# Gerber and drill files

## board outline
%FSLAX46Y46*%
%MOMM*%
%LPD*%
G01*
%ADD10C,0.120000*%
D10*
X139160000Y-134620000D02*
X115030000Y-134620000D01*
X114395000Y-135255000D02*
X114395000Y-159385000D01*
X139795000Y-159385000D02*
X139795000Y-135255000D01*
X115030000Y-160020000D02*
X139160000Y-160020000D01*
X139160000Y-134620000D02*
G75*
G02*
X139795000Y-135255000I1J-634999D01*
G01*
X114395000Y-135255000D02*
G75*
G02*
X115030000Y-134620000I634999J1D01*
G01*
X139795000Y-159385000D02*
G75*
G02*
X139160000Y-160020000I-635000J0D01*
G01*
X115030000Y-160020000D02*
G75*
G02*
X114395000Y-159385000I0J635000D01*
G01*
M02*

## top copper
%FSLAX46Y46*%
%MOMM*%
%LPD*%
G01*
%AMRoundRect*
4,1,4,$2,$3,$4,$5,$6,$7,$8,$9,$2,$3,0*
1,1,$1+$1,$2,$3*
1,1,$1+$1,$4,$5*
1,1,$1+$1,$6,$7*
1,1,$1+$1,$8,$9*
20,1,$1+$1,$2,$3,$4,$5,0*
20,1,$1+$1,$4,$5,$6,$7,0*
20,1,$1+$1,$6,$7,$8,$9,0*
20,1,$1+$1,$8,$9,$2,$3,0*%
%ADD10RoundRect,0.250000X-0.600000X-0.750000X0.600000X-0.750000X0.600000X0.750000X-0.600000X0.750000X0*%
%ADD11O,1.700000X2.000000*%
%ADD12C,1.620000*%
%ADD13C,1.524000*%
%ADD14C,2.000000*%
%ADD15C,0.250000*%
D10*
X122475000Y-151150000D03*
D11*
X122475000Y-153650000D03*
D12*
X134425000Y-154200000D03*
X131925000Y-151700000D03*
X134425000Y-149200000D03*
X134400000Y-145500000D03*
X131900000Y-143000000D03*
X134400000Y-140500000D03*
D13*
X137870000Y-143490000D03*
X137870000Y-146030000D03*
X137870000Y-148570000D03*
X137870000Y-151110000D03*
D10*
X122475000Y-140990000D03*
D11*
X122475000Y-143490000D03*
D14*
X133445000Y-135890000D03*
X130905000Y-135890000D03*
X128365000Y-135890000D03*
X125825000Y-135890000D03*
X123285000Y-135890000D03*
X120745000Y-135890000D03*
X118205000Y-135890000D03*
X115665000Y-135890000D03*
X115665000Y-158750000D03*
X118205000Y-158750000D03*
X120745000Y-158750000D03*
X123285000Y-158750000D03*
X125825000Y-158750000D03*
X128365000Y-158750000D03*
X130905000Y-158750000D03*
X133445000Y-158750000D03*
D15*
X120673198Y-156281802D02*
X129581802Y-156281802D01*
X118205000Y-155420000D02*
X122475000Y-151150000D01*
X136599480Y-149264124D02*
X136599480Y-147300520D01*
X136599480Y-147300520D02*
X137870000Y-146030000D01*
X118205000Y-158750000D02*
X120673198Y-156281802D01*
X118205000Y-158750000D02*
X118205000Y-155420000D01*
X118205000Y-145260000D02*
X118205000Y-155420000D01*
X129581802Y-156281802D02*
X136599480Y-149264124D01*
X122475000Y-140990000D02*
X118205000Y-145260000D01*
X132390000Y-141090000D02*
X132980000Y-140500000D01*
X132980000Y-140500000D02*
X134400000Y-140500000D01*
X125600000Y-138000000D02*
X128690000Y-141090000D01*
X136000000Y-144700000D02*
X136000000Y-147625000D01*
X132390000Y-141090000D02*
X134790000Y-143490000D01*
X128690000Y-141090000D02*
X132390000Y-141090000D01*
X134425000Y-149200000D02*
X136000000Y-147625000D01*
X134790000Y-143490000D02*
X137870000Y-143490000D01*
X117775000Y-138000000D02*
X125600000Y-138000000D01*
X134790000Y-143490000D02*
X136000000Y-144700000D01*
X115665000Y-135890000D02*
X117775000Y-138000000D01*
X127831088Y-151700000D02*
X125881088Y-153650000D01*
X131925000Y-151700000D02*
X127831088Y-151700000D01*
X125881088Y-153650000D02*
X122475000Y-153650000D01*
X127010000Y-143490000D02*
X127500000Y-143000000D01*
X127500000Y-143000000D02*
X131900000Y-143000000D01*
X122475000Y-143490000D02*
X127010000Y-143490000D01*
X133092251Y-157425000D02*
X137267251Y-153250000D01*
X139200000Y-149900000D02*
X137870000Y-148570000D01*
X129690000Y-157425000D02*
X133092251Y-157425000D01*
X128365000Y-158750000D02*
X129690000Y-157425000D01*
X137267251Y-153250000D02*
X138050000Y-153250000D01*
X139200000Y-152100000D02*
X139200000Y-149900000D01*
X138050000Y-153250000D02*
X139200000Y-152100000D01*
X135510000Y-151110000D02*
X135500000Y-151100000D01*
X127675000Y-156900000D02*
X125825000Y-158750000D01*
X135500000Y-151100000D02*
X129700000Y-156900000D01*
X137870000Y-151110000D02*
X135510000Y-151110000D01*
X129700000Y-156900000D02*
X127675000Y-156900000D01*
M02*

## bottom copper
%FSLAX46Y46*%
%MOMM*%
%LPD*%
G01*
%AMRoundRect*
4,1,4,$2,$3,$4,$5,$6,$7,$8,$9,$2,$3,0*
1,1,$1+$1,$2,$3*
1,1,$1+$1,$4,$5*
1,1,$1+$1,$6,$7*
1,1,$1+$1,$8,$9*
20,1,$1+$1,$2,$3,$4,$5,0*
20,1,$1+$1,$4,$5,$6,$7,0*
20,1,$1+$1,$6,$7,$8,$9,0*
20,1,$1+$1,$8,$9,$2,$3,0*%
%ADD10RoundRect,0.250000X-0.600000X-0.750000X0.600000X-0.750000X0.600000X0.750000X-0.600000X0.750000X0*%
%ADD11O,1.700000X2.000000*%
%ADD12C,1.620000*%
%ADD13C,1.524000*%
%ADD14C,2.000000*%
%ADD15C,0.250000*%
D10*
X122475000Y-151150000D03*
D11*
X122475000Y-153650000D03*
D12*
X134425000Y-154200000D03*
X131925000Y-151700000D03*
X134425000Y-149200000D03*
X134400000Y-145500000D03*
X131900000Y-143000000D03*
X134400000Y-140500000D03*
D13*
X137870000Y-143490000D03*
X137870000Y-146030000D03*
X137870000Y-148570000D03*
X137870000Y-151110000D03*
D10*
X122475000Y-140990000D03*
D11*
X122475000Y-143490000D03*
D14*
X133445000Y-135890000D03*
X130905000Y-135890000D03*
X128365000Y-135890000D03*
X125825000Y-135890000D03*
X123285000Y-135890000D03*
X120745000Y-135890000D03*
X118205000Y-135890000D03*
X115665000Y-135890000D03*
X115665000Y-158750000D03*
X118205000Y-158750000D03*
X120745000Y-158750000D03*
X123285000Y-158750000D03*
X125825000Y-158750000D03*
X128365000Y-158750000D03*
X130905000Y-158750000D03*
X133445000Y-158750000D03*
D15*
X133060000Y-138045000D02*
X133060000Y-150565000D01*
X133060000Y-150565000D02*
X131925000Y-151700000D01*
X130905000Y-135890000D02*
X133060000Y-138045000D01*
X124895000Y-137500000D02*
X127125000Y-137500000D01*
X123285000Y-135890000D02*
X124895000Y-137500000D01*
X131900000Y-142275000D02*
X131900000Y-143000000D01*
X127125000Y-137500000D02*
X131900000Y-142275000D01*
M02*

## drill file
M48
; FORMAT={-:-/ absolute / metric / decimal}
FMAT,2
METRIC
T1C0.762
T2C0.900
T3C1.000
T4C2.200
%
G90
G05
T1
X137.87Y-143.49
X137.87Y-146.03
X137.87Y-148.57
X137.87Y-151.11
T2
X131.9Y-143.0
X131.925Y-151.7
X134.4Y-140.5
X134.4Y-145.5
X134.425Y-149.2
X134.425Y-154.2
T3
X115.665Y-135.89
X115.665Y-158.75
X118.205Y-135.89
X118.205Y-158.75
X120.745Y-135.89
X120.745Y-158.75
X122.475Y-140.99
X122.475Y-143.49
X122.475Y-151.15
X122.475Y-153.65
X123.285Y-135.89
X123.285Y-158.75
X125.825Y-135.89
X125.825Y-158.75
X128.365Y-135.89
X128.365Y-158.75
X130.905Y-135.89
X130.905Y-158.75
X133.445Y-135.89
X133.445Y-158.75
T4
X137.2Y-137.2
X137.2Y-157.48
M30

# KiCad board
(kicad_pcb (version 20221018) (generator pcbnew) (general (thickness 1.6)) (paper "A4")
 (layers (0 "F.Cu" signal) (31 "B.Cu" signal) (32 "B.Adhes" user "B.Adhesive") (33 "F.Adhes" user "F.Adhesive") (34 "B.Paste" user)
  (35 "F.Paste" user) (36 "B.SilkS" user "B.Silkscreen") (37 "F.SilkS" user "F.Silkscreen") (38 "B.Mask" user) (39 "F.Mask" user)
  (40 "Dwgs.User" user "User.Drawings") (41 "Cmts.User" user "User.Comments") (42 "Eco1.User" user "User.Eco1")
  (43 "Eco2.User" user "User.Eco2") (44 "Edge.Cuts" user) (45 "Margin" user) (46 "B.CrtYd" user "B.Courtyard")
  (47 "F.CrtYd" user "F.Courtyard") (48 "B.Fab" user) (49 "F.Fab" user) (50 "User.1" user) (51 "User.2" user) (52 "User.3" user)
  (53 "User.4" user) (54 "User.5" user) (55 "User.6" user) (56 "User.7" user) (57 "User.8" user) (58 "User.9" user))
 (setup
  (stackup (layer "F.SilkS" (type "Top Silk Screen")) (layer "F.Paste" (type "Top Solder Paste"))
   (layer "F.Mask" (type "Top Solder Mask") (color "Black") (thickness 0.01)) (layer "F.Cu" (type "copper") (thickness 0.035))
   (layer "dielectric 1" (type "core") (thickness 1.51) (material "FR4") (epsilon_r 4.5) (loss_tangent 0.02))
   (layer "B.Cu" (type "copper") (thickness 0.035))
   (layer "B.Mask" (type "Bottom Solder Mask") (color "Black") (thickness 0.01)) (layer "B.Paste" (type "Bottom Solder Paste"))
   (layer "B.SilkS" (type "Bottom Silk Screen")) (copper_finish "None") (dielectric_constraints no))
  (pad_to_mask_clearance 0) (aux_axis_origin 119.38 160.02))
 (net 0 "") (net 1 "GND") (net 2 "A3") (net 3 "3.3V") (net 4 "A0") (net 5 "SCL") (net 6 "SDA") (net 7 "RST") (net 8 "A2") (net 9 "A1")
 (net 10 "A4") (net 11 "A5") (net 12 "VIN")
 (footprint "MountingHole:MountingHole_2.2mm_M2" (layer "F.Cu") (at 137.2 137.2)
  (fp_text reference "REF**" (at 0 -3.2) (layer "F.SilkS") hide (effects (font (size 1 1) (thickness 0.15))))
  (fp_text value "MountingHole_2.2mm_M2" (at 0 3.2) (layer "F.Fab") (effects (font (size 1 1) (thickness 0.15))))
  (pad "" np_thru_hole circle (at 0 0) (size 2.2 2.2) (drill 2.2) (layers "*.Cu" "*.Mask")))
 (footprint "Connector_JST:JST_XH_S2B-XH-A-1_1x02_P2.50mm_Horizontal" (layer "F.Cu") (at 114.375 152.4 -90)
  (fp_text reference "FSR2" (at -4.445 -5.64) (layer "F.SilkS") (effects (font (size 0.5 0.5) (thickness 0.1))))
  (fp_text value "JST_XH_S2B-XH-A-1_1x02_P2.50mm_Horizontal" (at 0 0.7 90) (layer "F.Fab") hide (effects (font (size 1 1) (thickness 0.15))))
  (pad "1" thru_hole roundrect (at -1.25 -8.1) (size 1.7 2) (drill 1) (layers "*.Cu" "*.Mask") (roundrect_rratio 0.1470588235) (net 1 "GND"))
  (pad "2" thru_hole oval (at 1.25 -8.1) (size 1.7 2) (drill 1) (layers "*.Cu" "*.Mask") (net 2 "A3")))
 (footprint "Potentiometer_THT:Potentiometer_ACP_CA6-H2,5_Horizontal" (layer "F.Cu") (at 134.425 154.2 180)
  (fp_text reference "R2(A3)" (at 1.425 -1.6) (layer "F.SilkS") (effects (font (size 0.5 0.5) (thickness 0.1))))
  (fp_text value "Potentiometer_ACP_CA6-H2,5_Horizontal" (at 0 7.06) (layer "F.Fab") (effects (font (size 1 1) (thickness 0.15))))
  (pad "1" thru_hole circle (at 0 0 180) (size 1.62 1.62) (drill 0.9) (layers "*.Cu" "*.Mask"))
  (pad "2" thru_hole circle (at 2.5 2.5 180) (size 1.62 1.62) (drill 0.9) (layers "*.Cu" "*.Mask") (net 2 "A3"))
  (pad "3" thru_hole circle (at 0 5 180) (size 1.62 1.62) (drill 0.9) (layers "*.Cu" "*.Mask") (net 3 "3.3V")))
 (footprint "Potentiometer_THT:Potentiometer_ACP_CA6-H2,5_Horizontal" (layer "F.Cu") (at 134.4 145.5 180)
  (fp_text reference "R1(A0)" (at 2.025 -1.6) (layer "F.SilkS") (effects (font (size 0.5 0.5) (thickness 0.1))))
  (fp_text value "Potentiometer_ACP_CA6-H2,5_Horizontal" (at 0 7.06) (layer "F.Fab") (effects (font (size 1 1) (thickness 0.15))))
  (pad "1" thru_hole circle (at 0 0 180) (size 1.62 1.62) (drill 0.9) (layers "*.Cu" "*.Mask"))
  (pad "2" thru_hole circle (at 2.5 2.5 180) (size 1.62 1.62) (drill 0.9) (layers "*.Cu" "*.Mask") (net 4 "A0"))
  (pad "3" thru_hole circle (at 0 5 180) (size 1.62 1.62) (drill 0.9) (layers "*.Cu" "*.Mask") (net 3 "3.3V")))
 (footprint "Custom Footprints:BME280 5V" (layer "F.Cu") (at 136.6 147.3 -90)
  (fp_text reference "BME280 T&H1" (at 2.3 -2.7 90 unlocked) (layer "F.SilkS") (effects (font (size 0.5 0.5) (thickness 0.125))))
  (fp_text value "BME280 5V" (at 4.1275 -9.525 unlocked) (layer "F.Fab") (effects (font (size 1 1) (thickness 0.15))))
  (pad "1" thru_hole circle (at -3.81 -1.27 180) (size 1.524 1.524) (drill 0.762) (layers "*.Cu" "*.Mask") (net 3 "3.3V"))
  (pad "2" thru_hole circle (at -1.27 -1.27 180) (size 1.524 1.524) (drill 0.762) (layers "*.Cu" "*.Mask") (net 1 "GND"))
  (pad "3" thru_hole circle (at 1.27 -1.27 180) (size 1.524 1.524) (drill 0.762) (layers "*.Cu" "*.Mask") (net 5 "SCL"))
  (pad "4" thru_hole circle (at 3.81 -1.27 180) (size 1.524 1.524) (drill 0.762) (layers "*.Cu" "*.Mask") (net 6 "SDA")))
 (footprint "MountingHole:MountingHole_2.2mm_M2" (layer "F.Cu") (at 137.2 157.44)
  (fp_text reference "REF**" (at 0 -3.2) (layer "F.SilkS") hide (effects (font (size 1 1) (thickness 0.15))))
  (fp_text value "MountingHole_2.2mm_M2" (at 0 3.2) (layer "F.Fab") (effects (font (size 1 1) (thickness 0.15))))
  (pad "" np_thru_hole circle (at 0 0.04) (size 2.2 2.2) (drill 2.2) (layers "F&B.Cu" "*.Mask")))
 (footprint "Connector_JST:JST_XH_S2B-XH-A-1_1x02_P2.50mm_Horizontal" (layer "F.Cu") (at 114.375 142.24 -90)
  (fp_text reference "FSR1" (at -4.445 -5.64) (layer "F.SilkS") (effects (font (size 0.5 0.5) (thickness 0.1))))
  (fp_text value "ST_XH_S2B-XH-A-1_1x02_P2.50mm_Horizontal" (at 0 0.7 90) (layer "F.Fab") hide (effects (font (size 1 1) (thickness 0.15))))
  (pad "1" thru_hole roundrect (at -1.25 -8.1) (size 1.7 2) (drill 1) (layers "*.Cu" "*.Mask") (roundrect_rratio 0.1470588235) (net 1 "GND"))
  (pad "2" thru_hole oval (at 1.25 -8.1) (size 1.7 2) (drill 1) (layers "*.Cu" "*.Mask") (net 4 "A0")))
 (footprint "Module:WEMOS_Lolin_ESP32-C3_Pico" (layer "F.Cu") (at 114.395 147.32 -90)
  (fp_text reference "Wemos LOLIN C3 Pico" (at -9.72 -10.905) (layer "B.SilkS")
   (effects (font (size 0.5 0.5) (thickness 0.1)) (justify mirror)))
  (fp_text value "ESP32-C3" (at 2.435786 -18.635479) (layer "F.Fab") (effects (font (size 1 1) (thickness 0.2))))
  (fp_line (start -12.7 -24.765) (end -12.7 -0.635) (stroke (width 0.12) (type solid)) (layer "Edge.Cuts"))
  (fp_line (start -12.065 0) (end 12.065 0) (stroke (width 0.12) (type solid)) (layer "Edge.Cuts"))
  (fp_line (start 12.065 -25.4) (end -12.065 -25.4) (stroke (width 0.12) (type solid)) (layer "Edge.Cuts"))
  (fp_line (start 12.7 -0.635) (end 12.7 -24.765) (stroke (width 0.12) (type solid)) (layer "Edge.Cuts"))
  (fp_arc (start -12.7 -24.765) (mid -12.514013 -25.214013) (end -12.065 -25.4) (stroke (width 0.12) (type solid)) (layer "Edge.Cuts"))
  (fp_arc (start -12.065 0) (mid -12.514013 -0.185987) (end -12.7 -0.635) (stroke (width 0.12) (type solid)) (layer "Edge.Cuts"))
  (fp_arc (start 12.065 -25.4) (mid 12.514013 -25.214013) (end 12.7 -24.765) (stroke (width 0.12) (type solid)) (layer "Edge.Cuts"))
  (fp_arc (start 12.7 -0.635) (mid 12.514013 -0.185987) (end 12.065 0) (stroke (width 0.12) (type solid)) (layer "Edge.Cuts"))
  (pad "1" thru_hole circle (at -11.43 -19.05 270) (size 2 2) (drill 1) (layers "*.Cu" "*.Mask") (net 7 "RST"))
  (pad "2" thru_hole circle (at -11.43 -16.51 270) (size 2 2) (drill 1) (layers "*.Cu" "*.Mask") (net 2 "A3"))
  (pad "3" thru_hole circle (at -11.43 -13.97 270) (size 2 2) (drill 1) (layers "*.Cu" "*.Mask") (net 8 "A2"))
  (pad "4" thru_hole circle (at -11.43 -11.43 270) (size 2 2) (drill 1) (layers "*.Cu" "*.Mask") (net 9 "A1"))
  (pad "5" thru_hole circle (at -11.43 -8.89 270) (size 2 2) (drill 1) (layers "*.Cu" "*.Mask") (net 4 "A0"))
  (pad "6" thru_hole circle (at -11.43 -6.35 270) (size 2 2) (drill 1) (layers "*.Cu" "*.Mask") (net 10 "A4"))
  (pad "7" thru_hole circle (at -11.43 -3.81 270) (size 2 2) (drill 1) (layers "*.Cu" "*.Mask") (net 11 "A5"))
  (pad "8" thru_hole circle (at -11.43 -1.27 270) (size 2 2) (drill 1) (layers "*.Cu" "*.Mask") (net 3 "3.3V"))
  (pad "9" thru_hole circle (at 11.43 -1.27 270) (size 2 2) (drill 1) (layers "*.Cu" "*.Mask") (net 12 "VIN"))
  (pad "10" thru_hole circle (at 11.43 -3.81 270) (size 2 2) (drill 1) (layers "*.Cu" "*.Mask") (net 1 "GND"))
  (pad "11" thru_hole circle (at 11.43 -6.35 270) (size 2 2) (drill 1) (layers "*.Cu" "*.Mask"))
  (pad "12" thru_hole circle (at 11.43 -8.89 270) (size 2 2) (drill 1) (layers "*.Cu" "*.Mask"))
  (pad "13" thru_hole circle (at 11.43 -11.43 270) (size 2 2) (drill 1) (layers "*.Cu" "*.Mask") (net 6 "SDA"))
  (pad "14" thru_hole circle (at 11.43 -13.97 270) (size 2 2) (drill 1) (layers "*.Cu" "*.Mask") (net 5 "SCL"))
  (pad "15" thru_hole circle (at 11.43 -16.51 270) (size 2 2) (drill 1) (layers "*.Cu" "*.Mask"))
  (pad "16" thru_hole circle (at 11.43 -19.05 270) (size 2 2) (drill 1) (layers "*.Cu" "*.Mask")))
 (segment (start 120.673198 156.281802) (end 129.581802 156.281802) (width 0.25) (layer "F.Cu") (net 1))
 (segment (start 118.205 155.42) (end 122.475 151.15) (width 0.25) (layer "F.Cu") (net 1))
 (segment (start 136.59948 149.264124) (end 136.59948 147.30052) (width 0.25) (layer "F.Cu") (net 1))
 (segment (start 136.59948 147.30052) (end 137.87 146.03) (width 0.25) (layer "F.Cu") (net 1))
 (segment (start 118.205 158.75) (end 120.673198 156.281802) (width 0.25) (layer "F.Cu") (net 1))
 (segment (start 118.205 158.75) (end 118.205 155.42) (width 0.25) (layer "F.Cu") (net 1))
 (segment (start 118.205 145.26) (end 118.205 155.42) (width 0.25) (layer "F.Cu") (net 1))
 (segment (start 129.581802 156.281802) (end 136.59948 149.264124) (width 0.25) (layer "F.Cu") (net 1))
 (segment (start 122.475 140.99) (end 118.205 145.26) (width 0.25) (layer "F.Cu") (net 1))
 (segment (start 132.39 141.09) (end 132.98 140.5) (width 0.25) (layer "F.Cu") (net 3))
 (segment (start 132.98 140.5) (end 134.4 140.5) (width 0.25) (layer "F.Cu") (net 3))
 (segment (start 125.6 138) (end 128.69 141.09) (width 0.25) (layer "F.Cu") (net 3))
 (segment (start 136 144.7) (end 136 147.625) (width 0.25) (layer "F.Cu") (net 3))
 (segment (start 132.39 141.09) (end 134.79 143.49) (width 0.25) (layer "F.Cu") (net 3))
 (segment (start 128.69 141.09) (end 132.39 141.09) (width 0.25) (layer "F.Cu") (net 3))
 (segment (start 134.425 149.2) (end 136 147.625) (width 0.25) (layer "F.Cu") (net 3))
 (segment (start 134.79 143.49) (end 137.87 143.49) (width 0.25) (layer "F.Cu") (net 3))
 (segment (start 117.775 138) (end 125.6 138) (width 0.25) (layer "F.Cu") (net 3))
 (segment (start 134.79 143.49) (end 136 144.7) (width 0.25) (layer "F.Cu") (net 3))
 (segment (start 115.665 135.89) (end 117.775 138) (width 0.25) (layer "F.Cu") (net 3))
 (segment (start 127.831088 151.7) (end 125.881088 153.65) (width 0.25) (layer "F.Cu") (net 2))
 (segment (start 131.925 151.7) (end 127.831088 151.7) (width 0.25) (layer "F.Cu") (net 2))
 (segment (start 125.881088 153.65) (end 122.475 153.65) (width 0.25) (layer "F.Cu") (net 2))
 (segment (start 133.06 138.045) (end 133.06 150.565) (width 0.25) (layer "B.Cu") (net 2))
 (segment (start 133.06 150.565) (end 131.925 151.7) (width 0.25) (layer "B.Cu") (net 2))
 (segment (start 130.905 135.89) (end 133.06 138.045) (width 0.25) (layer "B.Cu") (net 2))
 (segment (start 127.01 143.49) (end 127.5 143) (width 0.25) (layer "F.Cu") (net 4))
 (segment (start 127.5 143) (end 131.9 143) (width 0.25) (layer "F.Cu") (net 4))
 (segment (start 122.475 143.49) (end 127.01 143.49) (width 0.25) (layer "F.Cu") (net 4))
 (segment (start 124.895 137.5) (end 127.125 137.5) (width 0.25) (layer "B.Cu") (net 4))
 (segment (start 123.285 135.89) (end 124.895 137.5) (width 0.25) (layer "B.Cu") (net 4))
 (segment (start 131.9 142.275) (end 131.9 143) (width 0.25) (layer "B.Cu") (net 4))
 (segment (start 127.125 137.5) (end 131.9 142.275) (width 0.25) (layer "B.Cu") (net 4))
 (segment (start 133.092251 157.425) (end 137.267251 153.25) (width 0.25) (layer "F.Cu") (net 5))
 (segment (start 139.2 149.9) (end 137.87 148.57) (width 0.25) (layer "F.Cu") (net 5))
 (segment (start 129.69 157.425) (end 133.092251 157.425) (width 0.25) (layer "F.Cu") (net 5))
 (segment (start 128.365 158.75) (end 129.69 157.425) (width 0.25) (layer "F.Cu") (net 5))
 (segment (start 137.267251 153.25) (end 138.05 153.25) (width 0.25) (layer "F.Cu") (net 5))
 (segment (start 139.2 152.1) (end 139.2 149.9) (width 0.25) (layer "F.Cu") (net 5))
 (segment (start 138.05 153.25) (end 139.2 152.1) (width 0.25) (layer "F.Cu") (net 5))
 (segment (start 135.51 151.11) (end 135.5 151.1) (width 0.25) (layer "F.Cu") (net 6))
 (segment (start 127.675 156.9) (end 125.825 158.75) (width 0.25) (layer "F.Cu") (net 6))
 (segment (start 135.5 151.1) (end 129.7 156.9) (width 0.25) (layer "F.Cu") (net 6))
 (segment (start 137.87 151.11) (end 135.51 151.11) (width 0.25) (layer "F.Cu") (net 6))
 (segment (start 129.7 156.9) (end 127.675 156.9) (width 0.25) (layer "F.Cu") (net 6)))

